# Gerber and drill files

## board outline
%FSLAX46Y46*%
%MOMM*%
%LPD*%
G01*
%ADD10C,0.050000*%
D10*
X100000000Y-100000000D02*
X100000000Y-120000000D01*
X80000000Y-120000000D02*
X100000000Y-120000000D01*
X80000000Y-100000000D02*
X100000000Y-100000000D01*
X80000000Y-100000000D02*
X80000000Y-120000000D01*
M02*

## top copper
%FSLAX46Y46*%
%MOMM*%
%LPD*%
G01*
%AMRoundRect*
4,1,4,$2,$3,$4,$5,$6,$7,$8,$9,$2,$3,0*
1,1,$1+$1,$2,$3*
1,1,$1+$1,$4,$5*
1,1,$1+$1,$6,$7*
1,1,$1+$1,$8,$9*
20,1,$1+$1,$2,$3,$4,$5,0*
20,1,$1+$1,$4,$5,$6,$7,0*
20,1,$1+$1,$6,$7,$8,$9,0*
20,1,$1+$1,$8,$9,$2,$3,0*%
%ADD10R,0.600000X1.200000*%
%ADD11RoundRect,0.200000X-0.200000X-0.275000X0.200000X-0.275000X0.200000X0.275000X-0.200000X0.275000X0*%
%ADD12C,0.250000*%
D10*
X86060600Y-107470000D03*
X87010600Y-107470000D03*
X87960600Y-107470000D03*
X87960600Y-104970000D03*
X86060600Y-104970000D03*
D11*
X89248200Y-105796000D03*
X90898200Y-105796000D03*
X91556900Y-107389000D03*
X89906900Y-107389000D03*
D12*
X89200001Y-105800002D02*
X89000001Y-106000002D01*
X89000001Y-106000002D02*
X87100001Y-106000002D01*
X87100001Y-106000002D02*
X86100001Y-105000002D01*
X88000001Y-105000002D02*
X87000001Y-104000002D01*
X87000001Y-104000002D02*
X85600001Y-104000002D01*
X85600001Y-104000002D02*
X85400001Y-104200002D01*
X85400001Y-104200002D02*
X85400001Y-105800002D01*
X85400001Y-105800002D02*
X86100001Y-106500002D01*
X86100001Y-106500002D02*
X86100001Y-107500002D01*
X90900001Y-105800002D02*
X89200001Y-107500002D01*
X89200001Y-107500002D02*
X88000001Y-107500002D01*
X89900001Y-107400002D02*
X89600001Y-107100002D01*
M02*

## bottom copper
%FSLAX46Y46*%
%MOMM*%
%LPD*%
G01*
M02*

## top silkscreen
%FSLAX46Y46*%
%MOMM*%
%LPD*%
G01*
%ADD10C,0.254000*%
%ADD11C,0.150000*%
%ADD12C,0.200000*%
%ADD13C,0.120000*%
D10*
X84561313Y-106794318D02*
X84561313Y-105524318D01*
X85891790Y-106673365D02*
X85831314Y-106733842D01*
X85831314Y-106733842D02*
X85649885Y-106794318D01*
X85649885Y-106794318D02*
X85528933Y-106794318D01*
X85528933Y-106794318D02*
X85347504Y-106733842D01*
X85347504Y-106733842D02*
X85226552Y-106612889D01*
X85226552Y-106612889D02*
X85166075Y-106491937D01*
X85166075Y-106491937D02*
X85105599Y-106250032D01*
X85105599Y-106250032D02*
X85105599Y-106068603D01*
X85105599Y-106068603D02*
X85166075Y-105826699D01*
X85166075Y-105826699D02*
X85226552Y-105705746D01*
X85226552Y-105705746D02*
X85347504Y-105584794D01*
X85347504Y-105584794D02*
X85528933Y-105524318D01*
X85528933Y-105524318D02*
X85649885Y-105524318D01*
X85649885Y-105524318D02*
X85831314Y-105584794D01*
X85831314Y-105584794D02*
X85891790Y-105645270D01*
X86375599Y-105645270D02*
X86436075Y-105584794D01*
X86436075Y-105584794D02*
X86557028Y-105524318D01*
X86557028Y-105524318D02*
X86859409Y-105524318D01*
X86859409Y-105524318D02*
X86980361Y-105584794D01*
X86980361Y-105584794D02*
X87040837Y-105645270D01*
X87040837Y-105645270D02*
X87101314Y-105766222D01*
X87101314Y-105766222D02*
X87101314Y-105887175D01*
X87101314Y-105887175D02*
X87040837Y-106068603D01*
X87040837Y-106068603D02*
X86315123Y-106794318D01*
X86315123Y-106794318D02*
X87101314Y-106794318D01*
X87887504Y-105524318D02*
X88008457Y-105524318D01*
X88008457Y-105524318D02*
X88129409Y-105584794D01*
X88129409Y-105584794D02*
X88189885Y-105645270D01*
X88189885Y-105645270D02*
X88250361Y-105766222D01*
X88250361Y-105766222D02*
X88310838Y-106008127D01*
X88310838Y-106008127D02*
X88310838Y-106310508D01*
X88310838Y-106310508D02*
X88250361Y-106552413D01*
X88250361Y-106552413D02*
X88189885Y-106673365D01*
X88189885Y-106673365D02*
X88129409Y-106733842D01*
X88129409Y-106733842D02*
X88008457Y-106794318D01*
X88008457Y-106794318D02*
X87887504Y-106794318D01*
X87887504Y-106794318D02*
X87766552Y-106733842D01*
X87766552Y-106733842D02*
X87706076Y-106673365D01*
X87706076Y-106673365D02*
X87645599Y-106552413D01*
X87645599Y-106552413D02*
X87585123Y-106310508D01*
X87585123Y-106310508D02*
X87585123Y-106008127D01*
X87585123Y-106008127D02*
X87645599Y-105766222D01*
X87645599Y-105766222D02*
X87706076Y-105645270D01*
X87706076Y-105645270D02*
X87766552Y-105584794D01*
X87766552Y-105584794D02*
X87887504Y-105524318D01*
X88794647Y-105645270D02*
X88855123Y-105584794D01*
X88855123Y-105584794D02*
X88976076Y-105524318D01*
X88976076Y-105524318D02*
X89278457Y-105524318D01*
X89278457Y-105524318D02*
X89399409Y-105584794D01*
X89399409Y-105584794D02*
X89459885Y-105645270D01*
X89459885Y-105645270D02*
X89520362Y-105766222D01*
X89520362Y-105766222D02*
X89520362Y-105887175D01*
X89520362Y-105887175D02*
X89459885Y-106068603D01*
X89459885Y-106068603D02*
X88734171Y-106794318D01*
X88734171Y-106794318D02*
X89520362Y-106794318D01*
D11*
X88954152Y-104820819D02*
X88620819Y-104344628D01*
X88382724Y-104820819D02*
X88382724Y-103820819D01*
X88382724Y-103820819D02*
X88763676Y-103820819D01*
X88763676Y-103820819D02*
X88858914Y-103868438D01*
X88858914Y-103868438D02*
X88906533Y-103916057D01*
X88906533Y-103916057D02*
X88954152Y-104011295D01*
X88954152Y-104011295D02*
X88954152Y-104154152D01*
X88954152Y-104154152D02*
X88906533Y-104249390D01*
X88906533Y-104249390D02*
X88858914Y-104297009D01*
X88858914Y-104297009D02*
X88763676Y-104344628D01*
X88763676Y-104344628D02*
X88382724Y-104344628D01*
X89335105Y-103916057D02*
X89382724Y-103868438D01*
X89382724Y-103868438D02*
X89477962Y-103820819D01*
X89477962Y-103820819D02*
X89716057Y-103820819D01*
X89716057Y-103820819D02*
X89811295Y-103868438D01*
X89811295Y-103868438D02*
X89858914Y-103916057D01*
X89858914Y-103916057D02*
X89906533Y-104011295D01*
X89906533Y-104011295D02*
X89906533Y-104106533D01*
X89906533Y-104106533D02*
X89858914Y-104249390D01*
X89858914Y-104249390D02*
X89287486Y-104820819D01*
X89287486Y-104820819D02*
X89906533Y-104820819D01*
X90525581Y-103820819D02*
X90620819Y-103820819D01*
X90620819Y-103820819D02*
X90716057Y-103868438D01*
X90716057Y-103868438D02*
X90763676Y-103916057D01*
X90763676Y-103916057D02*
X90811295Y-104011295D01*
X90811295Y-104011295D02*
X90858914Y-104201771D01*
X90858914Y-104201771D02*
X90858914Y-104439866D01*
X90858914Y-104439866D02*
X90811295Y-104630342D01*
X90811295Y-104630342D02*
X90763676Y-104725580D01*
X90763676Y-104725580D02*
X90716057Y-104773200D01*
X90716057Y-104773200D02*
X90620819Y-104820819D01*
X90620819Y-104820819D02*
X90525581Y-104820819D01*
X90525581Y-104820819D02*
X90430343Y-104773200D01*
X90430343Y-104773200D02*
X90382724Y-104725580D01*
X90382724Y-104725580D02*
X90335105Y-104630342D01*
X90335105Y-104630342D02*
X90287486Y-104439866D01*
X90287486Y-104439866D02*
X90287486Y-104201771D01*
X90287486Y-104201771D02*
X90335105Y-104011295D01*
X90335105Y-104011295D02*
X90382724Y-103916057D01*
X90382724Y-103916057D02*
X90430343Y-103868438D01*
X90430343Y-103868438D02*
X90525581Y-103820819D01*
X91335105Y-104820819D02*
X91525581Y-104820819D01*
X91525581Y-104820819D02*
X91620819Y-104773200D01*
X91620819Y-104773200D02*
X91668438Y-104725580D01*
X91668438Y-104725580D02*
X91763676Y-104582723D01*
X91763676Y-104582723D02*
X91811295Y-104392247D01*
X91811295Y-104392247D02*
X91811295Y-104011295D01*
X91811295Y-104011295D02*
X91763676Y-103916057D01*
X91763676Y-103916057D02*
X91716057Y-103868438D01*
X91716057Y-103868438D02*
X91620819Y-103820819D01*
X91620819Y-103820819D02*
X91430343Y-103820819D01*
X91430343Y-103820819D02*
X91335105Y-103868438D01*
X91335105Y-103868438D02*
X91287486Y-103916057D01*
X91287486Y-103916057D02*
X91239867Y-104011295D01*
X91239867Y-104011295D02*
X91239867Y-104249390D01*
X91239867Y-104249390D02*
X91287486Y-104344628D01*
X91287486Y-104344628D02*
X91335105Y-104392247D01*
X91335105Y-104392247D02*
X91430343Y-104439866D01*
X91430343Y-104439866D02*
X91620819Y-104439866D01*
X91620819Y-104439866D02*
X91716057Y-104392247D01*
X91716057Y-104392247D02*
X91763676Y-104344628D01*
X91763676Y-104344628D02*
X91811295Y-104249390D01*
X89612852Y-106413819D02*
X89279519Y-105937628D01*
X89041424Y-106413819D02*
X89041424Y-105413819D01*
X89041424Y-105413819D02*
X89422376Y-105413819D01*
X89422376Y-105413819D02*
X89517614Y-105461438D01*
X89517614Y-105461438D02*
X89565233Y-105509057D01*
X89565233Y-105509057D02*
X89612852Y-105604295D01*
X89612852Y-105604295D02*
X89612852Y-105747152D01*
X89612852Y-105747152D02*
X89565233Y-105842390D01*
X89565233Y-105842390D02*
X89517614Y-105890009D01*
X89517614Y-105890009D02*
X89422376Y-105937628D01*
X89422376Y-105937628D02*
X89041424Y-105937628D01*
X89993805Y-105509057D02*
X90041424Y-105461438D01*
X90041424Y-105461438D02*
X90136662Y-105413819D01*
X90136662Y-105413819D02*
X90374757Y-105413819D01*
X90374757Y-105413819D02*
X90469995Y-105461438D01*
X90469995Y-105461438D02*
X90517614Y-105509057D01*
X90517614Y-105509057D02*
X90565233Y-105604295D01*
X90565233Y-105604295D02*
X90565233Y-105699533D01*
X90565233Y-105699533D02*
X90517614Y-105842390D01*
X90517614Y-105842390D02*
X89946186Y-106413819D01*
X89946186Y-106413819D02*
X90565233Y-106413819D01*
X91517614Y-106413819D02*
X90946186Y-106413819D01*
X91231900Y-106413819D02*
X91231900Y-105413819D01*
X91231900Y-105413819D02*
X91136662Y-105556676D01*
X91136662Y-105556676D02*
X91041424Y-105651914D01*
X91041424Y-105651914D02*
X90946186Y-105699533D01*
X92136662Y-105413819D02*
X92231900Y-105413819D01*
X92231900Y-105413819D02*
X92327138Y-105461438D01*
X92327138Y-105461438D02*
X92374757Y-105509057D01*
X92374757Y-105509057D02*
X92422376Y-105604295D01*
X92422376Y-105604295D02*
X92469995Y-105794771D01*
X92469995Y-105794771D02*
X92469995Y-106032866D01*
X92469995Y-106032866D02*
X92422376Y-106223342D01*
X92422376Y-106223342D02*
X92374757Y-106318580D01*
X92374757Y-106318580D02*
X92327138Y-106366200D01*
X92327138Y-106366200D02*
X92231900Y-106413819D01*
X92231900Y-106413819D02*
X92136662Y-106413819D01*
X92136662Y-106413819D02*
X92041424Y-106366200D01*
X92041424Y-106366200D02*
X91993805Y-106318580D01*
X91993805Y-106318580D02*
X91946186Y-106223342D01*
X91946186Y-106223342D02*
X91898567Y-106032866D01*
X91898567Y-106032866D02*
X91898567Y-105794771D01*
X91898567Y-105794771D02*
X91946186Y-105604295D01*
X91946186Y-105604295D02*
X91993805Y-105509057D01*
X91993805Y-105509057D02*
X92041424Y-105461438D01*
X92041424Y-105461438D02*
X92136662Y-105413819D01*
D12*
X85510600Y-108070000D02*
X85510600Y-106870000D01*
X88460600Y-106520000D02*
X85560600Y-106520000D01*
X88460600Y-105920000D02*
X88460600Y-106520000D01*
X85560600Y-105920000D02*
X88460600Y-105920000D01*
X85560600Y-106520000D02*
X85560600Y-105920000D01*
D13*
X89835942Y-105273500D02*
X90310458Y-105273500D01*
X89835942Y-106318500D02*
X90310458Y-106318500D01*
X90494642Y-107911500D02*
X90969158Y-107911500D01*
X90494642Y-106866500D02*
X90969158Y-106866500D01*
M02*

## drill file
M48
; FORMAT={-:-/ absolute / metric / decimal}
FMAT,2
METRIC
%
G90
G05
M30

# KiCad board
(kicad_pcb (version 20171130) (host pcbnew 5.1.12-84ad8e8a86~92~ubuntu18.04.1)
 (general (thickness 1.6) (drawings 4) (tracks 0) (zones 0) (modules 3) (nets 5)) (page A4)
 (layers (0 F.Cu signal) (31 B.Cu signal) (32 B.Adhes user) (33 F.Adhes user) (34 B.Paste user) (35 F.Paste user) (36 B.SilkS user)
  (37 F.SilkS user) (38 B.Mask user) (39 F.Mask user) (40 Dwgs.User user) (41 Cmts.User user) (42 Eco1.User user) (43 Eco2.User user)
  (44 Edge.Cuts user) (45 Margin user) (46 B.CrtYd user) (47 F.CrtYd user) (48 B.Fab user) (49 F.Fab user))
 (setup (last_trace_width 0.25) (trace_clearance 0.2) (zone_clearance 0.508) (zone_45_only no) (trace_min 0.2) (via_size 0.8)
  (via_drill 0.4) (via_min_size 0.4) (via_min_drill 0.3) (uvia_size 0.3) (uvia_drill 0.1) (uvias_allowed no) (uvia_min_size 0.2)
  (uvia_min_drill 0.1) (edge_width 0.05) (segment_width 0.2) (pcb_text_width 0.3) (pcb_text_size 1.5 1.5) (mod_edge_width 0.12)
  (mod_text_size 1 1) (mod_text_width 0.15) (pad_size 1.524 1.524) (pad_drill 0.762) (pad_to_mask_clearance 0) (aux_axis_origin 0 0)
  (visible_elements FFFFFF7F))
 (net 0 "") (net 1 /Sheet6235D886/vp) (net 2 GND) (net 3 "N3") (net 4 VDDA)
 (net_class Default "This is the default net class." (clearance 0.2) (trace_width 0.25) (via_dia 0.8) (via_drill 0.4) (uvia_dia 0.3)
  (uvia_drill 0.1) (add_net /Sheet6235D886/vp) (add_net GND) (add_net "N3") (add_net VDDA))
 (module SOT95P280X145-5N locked (layer F.Cu) (at 87.010600 106.220000 90.000000)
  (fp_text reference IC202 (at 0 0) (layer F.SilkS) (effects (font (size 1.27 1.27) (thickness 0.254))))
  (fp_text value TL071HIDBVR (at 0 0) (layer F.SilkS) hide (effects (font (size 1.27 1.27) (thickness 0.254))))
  (fp_line (start -1.85 -1.5) (end -0.65 -1.5) (layer F.SilkS) (width 0.2))
  (fp_line (start -0.3 1.45) (end -0.3 -1.45) (layer F.SilkS) (width 0.2))
  (fp_line (start 0.3 1.45) (end -0.3 1.45) (layer F.SilkS) (width 0.2))
  (fp_line (start 0.3 -1.45) (end 0.3 1.45) (layer F.SilkS) (width 0.2))
  (fp_line (start -0.3 -1.45) (end 0.3 -1.45) (layer F.SilkS) (width 0.2))
  (pad 1 smd rect (at -1.25 -0.95 180.000000) (size 0.6 1.2) (layers F.Cu F.Mask F.Paste) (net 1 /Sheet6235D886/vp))
  (pad 2 smd rect (at -1.25 0 180.000000) (size 0.6 1.2) (layers F.Cu F.Mask F.Paste) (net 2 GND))
  (pad 3 smd rect (at -1.25 0.95 180.000000) (size 0.6 1.2) (layers F.Cu F.Mask F.Paste) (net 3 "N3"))
  (pad 4 smd rect (at 1.25 0.95 180.000000) (size 0.6 1.2) (layers F.Cu F.Mask F.Paste) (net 1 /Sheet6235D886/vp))
  (pad 5 smd rect (at 1.25 -0.95 180.000000) (size 0.6 1.2) (layers F.Cu F.Mask F.Paste) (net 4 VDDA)))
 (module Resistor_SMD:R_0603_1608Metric (layer F.Cu) (at 90.073200 105.796000)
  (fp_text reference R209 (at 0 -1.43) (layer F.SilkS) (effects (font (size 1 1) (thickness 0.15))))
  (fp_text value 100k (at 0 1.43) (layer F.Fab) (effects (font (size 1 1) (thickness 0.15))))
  (fp_line (start -0.237258 -0.5225) (end 0.237258 -0.5225) (layer F.SilkS) (width 0.12))
  (fp_line (start -0.237258 0.5225) (end 0.237258 0.5225) (layer F.SilkS) (width 0.12))
  (pad 1 smd roundrect (at -0.825 0) (size 0.8 0.95) (layers F.Cu F.Mask F.Paste) (roundrect_rratio 0.25) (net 4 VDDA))
  (pad 2 smd roundrect (at 0.825 0) (size 0.8 0.95) (layers F.Cu F.Mask F.Paste) (roundrect_rratio 0.25) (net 3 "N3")))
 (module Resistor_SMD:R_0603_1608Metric (layer F.Cu) (at 90.731900 107.389000)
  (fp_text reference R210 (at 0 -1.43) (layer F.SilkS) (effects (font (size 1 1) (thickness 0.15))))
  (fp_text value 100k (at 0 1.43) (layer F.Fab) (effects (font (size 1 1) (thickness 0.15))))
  (fp_line (start -0.237258 0.5225) (end 0.237258 0.5225) (layer F.SilkS) (width 0.12))
  (fp_line (start -0.237258 -0.5225) (end 0.237258 -0.5225) (layer F.SilkS) (width 0.12))
  (pad 2 smd roundrect (at 0.825 0) (size 0.8 0.95) (layers F.Cu F.Mask F.Paste) (roundrect_rratio 0.25) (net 2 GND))
  (pad 1 smd roundrect (at -0.825 0) (size 0.8 0.95) (layers F.Cu F.Mask F.Paste) (roundrect_rratio 0.25) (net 3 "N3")))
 (gr_line (start 100 100) (end 100 120) (layer Edge.Cuts) (width 0.05))
 (gr_line (start 80 120) (end 100 120) (layer Edge.Cuts) (width 0.05))
 (gr_line (start 80 100) (end 100 100) (layer Edge.Cuts) (width 0.05))
 (gr_line (start 80 100) (end 80 120) (layer Edge.Cuts) (width 0.05))
 (segment (start 89.200001 105.800002) (end 89.000001 106.000002) (width 0.250000) (layer F.Cu) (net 4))
 (segment (start 89.000001 106.000002) (end 87.100001 106.000002) (width 0.250000) (layer F.Cu) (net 4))
 (segment (start 87.100001 106.000002) (end 86.100001 105.000002) (width 0.250000) (layer F.Cu) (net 4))
 (segment (start 88.000001 105.000002) (end 87.000001 104.000002) (width 0.250000) (layer F.Cu) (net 1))
 (segment (start 87.000001 104.000002) (end 85.600001 104.000002) (width 0.250000) (layer F.Cu) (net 1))
 (segment (start 85.600001 104.000002) (end 85.400001 104.200002) (width 0.250000) (layer F.Cu) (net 1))
 (segment (start 85.400001 104.200002) (end 85.400001 105.800002) (width 0.250000) (layer F.Cu) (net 1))
 (segment (start 85.400001 105.800002) (end 86.100001 106.500002) (width 0.250000) (layer F.Cu) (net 1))
 (segment (start 86.100001 106.500002) (end 86.100001 107.500002) (width 0.250000) (layer F.Cu) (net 1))
 (segment (start 90.900001 105.800002) (end 89.200001 107.500002) (width 0.250000) (layer F.Cu) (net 3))
 (segment (start 89.200001 107.500002) (end 88.000001 107.500002) (width 0.250000) (layer F.Cu) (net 3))
 (segment (start 89.900001 107.400002) (end 89.600001 107.100002) (width 0.250000) (layer F.Cu) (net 3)))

